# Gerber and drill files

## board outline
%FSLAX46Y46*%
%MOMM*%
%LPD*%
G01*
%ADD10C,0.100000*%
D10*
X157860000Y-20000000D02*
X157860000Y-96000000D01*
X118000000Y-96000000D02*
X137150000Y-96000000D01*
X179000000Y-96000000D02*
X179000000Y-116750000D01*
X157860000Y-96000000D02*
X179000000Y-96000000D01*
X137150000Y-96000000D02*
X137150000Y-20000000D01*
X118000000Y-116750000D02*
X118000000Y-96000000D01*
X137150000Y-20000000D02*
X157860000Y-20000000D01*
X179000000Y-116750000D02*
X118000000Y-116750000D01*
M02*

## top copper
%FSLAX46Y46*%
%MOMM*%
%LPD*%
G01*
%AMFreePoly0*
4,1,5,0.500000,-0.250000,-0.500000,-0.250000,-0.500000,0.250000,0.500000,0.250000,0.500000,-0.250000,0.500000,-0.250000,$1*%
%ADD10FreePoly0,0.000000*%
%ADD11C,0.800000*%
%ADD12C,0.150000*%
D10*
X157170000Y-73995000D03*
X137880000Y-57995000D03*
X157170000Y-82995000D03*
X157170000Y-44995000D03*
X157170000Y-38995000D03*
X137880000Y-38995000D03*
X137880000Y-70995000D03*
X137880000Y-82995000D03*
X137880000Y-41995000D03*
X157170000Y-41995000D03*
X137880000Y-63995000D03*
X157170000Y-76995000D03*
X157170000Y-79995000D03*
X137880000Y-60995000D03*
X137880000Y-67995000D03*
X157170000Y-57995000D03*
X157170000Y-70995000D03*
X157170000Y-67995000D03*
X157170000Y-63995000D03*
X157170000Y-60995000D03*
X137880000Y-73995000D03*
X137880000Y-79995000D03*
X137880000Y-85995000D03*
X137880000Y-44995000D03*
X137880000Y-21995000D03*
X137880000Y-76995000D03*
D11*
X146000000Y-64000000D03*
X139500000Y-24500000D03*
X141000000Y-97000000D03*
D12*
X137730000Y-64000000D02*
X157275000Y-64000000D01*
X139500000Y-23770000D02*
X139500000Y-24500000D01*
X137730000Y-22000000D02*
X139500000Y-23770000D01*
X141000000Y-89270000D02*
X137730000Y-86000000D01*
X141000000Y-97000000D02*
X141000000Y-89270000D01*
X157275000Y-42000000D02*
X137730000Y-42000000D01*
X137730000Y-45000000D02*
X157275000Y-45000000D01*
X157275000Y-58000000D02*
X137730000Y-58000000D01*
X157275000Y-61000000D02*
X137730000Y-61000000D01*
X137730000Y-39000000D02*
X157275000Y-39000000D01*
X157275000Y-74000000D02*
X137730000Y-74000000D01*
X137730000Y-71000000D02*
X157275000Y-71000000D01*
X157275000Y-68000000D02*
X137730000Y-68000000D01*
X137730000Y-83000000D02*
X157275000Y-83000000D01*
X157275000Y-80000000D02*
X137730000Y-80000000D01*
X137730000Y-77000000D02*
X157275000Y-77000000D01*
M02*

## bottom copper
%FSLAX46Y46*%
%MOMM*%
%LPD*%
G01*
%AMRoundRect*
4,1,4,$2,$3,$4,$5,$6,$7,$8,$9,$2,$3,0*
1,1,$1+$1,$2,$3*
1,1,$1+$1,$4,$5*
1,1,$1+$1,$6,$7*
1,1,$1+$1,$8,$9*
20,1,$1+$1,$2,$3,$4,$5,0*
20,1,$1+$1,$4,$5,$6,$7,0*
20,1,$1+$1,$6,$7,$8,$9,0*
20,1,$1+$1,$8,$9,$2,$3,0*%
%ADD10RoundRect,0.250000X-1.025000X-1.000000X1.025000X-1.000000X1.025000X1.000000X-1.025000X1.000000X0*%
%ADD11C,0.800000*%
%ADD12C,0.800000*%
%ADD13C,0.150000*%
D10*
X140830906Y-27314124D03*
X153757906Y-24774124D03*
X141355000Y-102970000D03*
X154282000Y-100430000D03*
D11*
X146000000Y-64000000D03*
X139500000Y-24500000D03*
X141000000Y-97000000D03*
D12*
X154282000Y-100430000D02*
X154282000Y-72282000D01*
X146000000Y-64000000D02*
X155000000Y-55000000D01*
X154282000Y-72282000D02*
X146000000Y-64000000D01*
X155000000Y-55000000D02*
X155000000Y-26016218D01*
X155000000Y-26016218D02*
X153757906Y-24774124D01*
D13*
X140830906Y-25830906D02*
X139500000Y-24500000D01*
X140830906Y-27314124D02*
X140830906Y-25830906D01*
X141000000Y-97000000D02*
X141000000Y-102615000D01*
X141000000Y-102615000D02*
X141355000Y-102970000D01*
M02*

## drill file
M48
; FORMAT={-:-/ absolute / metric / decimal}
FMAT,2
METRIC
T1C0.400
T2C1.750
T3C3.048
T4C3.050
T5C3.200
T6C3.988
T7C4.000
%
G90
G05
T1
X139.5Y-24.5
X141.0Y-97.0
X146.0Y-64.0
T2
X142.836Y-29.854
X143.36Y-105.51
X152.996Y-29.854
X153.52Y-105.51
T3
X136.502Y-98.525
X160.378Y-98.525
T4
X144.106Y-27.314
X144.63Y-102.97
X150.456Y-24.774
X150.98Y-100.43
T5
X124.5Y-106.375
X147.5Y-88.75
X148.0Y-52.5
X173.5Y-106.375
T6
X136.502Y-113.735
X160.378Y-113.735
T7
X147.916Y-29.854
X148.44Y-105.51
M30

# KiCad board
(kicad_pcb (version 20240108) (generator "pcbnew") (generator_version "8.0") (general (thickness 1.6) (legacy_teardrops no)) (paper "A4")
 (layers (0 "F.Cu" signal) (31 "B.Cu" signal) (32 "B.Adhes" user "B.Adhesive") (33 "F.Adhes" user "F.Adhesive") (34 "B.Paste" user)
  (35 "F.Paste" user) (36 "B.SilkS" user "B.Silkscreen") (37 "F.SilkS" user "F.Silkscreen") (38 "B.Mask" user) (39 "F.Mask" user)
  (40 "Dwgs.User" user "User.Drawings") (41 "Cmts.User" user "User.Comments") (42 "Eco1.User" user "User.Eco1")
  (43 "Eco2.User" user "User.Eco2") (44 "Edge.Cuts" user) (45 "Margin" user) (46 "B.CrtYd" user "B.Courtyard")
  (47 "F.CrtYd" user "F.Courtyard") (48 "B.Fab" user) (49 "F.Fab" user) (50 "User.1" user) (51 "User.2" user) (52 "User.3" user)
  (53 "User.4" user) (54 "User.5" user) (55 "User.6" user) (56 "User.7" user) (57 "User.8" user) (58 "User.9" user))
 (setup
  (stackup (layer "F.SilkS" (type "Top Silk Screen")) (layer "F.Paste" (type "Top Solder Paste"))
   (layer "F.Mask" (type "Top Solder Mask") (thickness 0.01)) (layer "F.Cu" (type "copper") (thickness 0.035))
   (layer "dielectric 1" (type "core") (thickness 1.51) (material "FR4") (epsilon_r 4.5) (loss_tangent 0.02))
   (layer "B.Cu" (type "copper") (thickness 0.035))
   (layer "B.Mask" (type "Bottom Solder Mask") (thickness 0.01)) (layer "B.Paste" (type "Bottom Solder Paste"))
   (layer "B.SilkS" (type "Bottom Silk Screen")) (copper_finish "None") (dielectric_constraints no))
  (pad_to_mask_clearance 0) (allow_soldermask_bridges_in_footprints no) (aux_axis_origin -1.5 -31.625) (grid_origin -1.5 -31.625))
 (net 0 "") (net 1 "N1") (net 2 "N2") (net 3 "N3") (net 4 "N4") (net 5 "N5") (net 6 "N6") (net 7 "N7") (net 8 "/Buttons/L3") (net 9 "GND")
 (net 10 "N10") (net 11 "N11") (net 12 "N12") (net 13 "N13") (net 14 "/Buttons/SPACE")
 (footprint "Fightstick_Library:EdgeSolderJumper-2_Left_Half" (layer "F.Cu") (at 157.82 73.995)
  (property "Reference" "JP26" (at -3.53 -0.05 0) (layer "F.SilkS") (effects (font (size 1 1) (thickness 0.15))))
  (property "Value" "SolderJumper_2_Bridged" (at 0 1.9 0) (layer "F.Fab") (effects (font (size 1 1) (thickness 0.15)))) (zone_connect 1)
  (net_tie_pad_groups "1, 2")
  (pad "1" smd custom (at -0.65 0) (size 1 0.5) (layers "F.Cu" "F.Mask") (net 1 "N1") (zone_connect 2) (thermal_bridge_angle 45)
   (options (clearance outline) (anchor rect)) (primitives)))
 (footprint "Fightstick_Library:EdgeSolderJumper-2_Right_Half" (layer "F.Cu") (at 137.23 57.995)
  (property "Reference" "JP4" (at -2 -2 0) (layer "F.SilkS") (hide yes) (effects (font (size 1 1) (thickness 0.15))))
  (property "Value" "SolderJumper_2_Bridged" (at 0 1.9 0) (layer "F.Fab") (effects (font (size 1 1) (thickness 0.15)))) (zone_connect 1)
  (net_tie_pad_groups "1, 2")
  (pad "2" smd custom (at 0.65 0) (size 1 0.5) (layers "F.Cu" "F.Mask") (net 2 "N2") (zone_connect 2) (thermal_bridge_angle 45)
   (options (clearance outline) (anchor rect)) (primitives)))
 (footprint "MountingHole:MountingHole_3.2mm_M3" (layer "F.Cu") (at 148 52.5 -90)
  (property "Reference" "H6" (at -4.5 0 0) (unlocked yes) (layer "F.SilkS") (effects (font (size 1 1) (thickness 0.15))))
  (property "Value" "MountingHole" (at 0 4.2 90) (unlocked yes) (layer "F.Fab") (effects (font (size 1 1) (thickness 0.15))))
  (pad "" np_thru_hole circle (at 0 0 270) (size 3.2 3.2) (drill 3.2) (layers "*.Cu" "*.Mask")))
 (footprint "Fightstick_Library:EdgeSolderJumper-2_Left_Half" (layer "F.Cu") (at 157.82 82.995)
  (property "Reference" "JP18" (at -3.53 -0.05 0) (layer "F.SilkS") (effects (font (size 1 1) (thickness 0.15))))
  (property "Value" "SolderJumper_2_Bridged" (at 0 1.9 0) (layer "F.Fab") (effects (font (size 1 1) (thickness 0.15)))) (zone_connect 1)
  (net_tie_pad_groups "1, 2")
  (pad "1" smd custom (at -0.65 0) (size 1 0.5) (layers "F.Cu" "F.Mask") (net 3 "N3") (zone_connect 2) (thermal_bridge_angle 45)
   (options (clearance outline) (anchor rect)) (primitives)))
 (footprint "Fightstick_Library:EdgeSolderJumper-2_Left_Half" (layer "F.Cu") (at 157.82 44.995)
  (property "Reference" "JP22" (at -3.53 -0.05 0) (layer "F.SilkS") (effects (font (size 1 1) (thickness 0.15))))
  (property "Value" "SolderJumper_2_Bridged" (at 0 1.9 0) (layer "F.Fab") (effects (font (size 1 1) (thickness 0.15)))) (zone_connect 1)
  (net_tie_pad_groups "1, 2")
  (pad "1" smd custom (at -0.65 0) (size 1 0.5) (layers "F.Cu" "F.Mask") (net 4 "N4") (zone_connect 2) (thermal_bridge_angle 45)
   (options (clearance outline) (anchor rect)) (primitives)))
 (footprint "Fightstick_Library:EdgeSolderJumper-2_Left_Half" (layer "F.Cu") (at 157.82 38.995)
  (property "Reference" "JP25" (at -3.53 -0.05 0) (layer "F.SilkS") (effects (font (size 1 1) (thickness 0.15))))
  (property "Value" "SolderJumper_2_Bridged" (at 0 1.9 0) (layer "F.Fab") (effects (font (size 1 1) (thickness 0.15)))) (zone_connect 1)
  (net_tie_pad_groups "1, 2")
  (pad "1" smd custom (at -0.65 0) (size 1 0.5) (layers "F.Cu" "F.Mask") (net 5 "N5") (zone_connect 2) (thermal_bridge_angle 45)
   (options (clearance outline) (anchor rect)) (primitives)))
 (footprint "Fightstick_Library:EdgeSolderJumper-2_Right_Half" (layer "F.Cu") (at 137.23 38.995)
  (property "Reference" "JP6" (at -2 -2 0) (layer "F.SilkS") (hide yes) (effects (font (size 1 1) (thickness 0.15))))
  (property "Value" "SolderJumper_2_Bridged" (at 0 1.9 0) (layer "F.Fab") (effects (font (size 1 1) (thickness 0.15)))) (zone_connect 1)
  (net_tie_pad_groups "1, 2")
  (pad "2" smd custom (at 0.65 0) (size 1 0.5) (layers "F.Cu" "F.Mask") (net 5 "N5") (zone_connect 2) (thermal_bridge_angle 45)
   (options (clearance outline) (anchor rect)) (primitives)))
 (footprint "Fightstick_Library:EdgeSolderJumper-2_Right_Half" (layer "F.Cu") (at 137.23 70.995)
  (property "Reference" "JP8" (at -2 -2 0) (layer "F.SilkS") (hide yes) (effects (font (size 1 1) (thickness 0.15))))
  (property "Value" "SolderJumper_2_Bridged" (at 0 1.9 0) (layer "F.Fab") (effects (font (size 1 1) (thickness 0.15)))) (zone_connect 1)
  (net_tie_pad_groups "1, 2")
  (pad "2" smd custom (at 0.65 0) (size 1 0.5) (layers "F.Cu" "F.Mask") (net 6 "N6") (zone_connect 2) (thermal_bridge_angle 45)
   (options (clearance outline) (anchor rect)) (primitives)))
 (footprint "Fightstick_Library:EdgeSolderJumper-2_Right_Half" (layer "F.Cu") (at 137.23 82.995)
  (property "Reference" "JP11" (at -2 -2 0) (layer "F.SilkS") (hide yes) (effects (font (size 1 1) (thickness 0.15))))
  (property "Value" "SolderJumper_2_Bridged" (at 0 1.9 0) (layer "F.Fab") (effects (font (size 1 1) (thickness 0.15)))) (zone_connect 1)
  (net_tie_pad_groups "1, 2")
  (pad "2" smd custom (at 0.65 0) (size 1 0.5) (layers "F.Cu" "F.Mask") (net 3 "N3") (zone_connect 2) (thermal_bridge_angle 45)
   (options (clearance outline) (anchor rect)) (primitives)))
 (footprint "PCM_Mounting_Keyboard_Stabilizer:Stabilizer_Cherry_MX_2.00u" (layer "F.Cu") (at 148.44 105.51)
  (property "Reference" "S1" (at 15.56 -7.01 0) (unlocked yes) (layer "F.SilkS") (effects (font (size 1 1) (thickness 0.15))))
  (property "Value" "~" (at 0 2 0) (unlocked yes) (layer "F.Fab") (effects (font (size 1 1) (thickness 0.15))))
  (pad "" np_thru_hole circle (at -11.938 -6.985) (size 3.048 3.048) (drill 3.048) (layers "*.Cu" "*.Mask"))
  (pad "" np_thru_hole circle (at -11.938 8.225) (size 3.9878 3.9878) (drill 3.9878) (layers "*.Cu" "*.Mask"))
  (pad "" np_thru_hole circle (at 11.938 -6.985) (size 3.048 3.048) (drill 3.048) (layers "*.Cu" "*.Mask"))
  (pad "" np_thru_hole circle (at 11.938 8.225) (size 3.9878 3.9878) (drill 3.9878) (layers "*.Cu" "*.Mask")))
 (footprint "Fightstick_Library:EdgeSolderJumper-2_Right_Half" (layer "F.Cu") (at 137.23 41.995)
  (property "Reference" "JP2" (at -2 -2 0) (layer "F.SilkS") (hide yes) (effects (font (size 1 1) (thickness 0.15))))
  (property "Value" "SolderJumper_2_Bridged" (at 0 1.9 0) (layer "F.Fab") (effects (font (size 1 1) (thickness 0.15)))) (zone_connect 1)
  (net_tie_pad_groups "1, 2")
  (pad "2" smd custom (at 0.65 0) (size 1 0.5) (layers "F.Cu" "F.Mask") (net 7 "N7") (zone_connect 2) (thermal_bridge_angle 45)
   (options (clearance outline) (anchor rect)) (primitives)))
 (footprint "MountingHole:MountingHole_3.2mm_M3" (layer "F.Cu") (at 147.5 88.75)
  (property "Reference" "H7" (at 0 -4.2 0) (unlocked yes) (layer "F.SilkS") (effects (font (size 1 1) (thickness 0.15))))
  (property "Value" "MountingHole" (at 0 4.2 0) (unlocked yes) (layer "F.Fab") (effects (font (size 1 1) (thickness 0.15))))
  (pad "" np_thru_hole circle (at 0 0) (size 3.2 3.2) (drill 3.2) (layers "*.Cu" "*.Mask")))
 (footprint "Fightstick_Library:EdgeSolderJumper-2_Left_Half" (layer "F.Cu") (at 157.82 41.995)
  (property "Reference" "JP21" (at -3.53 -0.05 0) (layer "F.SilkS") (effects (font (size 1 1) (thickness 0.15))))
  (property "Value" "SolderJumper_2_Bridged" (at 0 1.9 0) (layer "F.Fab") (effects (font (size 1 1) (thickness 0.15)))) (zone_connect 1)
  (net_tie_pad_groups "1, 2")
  (pad "1" smd custom (at -0.65 0) (size 1 0.5) (layers "F.Cu" "F.Mask") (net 7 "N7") (zone_connect 2) (thermal_bridge_angle 45)
   (options (clearance outline) (anchor rect)) (primitives)))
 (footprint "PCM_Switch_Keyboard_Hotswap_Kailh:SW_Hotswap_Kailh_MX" (layer "F.Cu") (at 147.915906 29.854124)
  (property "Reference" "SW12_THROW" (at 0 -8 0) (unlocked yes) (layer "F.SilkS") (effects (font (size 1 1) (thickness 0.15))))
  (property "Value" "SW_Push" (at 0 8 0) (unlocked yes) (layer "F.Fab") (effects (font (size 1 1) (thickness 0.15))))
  (pad "" np_thru_hole circle (at -5.08 0) (size 1.75 1.75) (drill 1.75) (layers "*.Cu" "*.Mask"))
  (pad "" np_thru_hole circle (at -3.81 -2.54) (size 3.05 3.05) (drill 3.05) (layers "*.Cu" "*.Mask"))
  (pad "" np_thru_hole circle (at 0 0) (size 4 4) (drill 4) (layers "*.Cu" "*.Mask"))
  (pad "" np_thru_hole circle (at 2.54 -5.08) (size 3.05 3.05) (drill 3.05) (layers "*.Cu" "*.Mask"))
  (pad "" np_thru_hole circle (at 5.08 0) (size 1.75 1.75) (drill 1.75) (layers "*.Cu" "*.Mask"))
  (pad "1" smd roundrect (at -7.085 -2.54) (size 2.55 2.5) (layers "B.Cu" "B.Paste" "B.Mask") (roundrect_rratio 0.1) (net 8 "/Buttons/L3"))
  (pad "2" smd roundrect (at 5.842 -5.08) (size 2.55 2.5) (layers "B.Cu" "B.Paste" "B.Mask") (roundrect_rratio 0.1) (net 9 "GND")))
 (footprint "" (layer "F.Cu") (at 173.5 106.375)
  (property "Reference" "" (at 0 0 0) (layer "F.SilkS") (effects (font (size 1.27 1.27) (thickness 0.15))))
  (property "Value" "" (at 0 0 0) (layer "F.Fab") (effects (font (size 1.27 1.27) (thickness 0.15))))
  (pad "" np_thru_hole circle (at 0 0 270) (size 3.2 3.2) (drill 3.2) (layers "F&B.Cu" "*.Mask")))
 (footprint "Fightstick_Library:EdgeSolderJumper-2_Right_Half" (layer "F.Cu") (at 137.23 63.995)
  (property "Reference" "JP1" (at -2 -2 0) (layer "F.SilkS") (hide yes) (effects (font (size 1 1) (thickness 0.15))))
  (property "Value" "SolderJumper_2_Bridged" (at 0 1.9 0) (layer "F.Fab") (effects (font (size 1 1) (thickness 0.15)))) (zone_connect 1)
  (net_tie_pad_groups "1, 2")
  (pad "2" smd custom (at 0.65 0) (size 1 0.5) (layers "F.Cu" "F.Mask") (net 9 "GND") (zone_connect 2) (thermal_bridge_angle 45)
   (options (clearance outline) (anchor rect)) (primitives)))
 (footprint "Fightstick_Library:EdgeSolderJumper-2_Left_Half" (layer "F.Cu") (at 157.82 76.995)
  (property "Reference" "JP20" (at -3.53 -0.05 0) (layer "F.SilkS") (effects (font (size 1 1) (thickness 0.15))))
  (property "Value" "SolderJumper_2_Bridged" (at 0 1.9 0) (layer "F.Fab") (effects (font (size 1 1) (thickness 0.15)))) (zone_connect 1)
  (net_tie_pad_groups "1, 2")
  (pad "1" smd custom (at -0.65 0) (size 1 0.5) (layers "F.Cu" "F.Mask") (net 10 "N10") (zone_connect 2) (thermal_bridge_angle 45)
   (options (clearance outline) (anchor rect)) (primitives)))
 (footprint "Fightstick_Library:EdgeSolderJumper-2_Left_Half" (layer "F.Cu") (at 157.82 79.995)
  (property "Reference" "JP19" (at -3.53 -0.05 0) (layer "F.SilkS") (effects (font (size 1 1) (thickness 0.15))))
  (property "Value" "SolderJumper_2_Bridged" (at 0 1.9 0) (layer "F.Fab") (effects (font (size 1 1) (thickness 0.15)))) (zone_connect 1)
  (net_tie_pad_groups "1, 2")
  (pad "1" smd custom (at -0.65 0) (size 1 0.5) (layers "F.Cu" "F.Mask") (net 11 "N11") (zone_connect 2) (thermal_bridge_angle 45)
   (options (clearance outline) (anchor rect)) (primitives)))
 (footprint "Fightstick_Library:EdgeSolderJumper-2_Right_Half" (layer "F.Cu") (at 137.23 60.995)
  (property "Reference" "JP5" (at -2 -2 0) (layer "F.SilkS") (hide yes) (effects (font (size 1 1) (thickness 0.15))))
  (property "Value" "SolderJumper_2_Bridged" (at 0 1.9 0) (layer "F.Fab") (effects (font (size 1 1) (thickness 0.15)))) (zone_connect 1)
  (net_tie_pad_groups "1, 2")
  (pad "2" smd custom (at 0.65 0) (size 1 0.5) (layers "F.Cu" "F.Mask") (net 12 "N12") (zone_connect 2) (thermal_bridge_angle 45)
   (options (clearance outline) (anchor rect)) (primitives)))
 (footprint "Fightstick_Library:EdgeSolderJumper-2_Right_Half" (layer "F.Cu") (at 137.23 67.995)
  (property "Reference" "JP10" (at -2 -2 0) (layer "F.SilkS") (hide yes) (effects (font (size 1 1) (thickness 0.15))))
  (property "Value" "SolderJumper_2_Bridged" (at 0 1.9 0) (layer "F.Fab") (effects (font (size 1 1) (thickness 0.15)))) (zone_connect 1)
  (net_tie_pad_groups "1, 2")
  (pad "2" smd custom (at 0.65 0) (size 1 0.5) (layers "F.Cu" "F.Mask") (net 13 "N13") (zone_connect 2) (thermal_bridge_angle 45)
   (options (clearance outline) (anchor rect)) (primitives)))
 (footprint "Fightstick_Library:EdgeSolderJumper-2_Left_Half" (layer "F.Cu") (at 157.82 57.995)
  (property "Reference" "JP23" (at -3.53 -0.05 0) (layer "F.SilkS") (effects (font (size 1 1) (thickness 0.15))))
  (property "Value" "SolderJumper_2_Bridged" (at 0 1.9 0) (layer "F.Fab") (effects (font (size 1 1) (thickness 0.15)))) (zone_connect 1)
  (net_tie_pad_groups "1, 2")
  (pad "1" smd custom (at -0.65 0) (size 1 0.5) (layers "F.Cu" "F.Mask") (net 2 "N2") (zone_connect 2) (thermal_bridge_angle 45)
   (options (clearance outline) (anchor rect)) (primitives)))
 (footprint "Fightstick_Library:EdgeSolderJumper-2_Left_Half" (layer "F.Cu") (at 157.82 70.995)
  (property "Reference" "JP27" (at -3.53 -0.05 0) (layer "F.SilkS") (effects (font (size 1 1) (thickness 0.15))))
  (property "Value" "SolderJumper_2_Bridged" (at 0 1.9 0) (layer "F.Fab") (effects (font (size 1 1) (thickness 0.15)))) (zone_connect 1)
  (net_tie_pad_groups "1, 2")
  (pad "1" smd custom (at -0.65 0) (size 1 0.5) (layers "F.Cu" "F.Mask") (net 6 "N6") (zone_connect 2) (thermal_bridge_angle 45)
   (options (clearance outline) (anchor rect)) (primitives)))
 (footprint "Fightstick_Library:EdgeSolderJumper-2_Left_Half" (layer "F.Cu") (at 157.82 67.995)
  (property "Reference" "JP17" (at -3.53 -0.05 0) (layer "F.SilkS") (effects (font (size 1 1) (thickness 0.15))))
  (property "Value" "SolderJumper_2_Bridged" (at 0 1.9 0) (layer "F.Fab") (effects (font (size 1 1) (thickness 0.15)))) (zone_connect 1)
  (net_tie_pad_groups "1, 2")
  (pad "1" smd custom (at -0.65 0) (size 1 0.5) (layers "F.Cu" "F.Mask") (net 13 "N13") (zone_connect 2) (thermal_bridge_angle 45)
   (options (clearance outline) (anchor rect)) (primitives)))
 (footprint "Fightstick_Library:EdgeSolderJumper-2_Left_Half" (layer "F.Cu") (at 157.82 63.995)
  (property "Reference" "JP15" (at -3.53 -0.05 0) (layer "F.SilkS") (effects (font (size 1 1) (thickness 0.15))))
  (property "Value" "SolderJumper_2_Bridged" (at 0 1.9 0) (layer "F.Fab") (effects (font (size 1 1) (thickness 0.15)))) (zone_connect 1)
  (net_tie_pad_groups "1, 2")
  (pad "1" smd custom (at -0.65 0) (size 1 0.5) (layers "F.Cu" "F.Mask") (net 9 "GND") (zone_connect 2) (thermal_bridge_angle 45)
   (options (clearance outline) (anchor rect)) (primitives)))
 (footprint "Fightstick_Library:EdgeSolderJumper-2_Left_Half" (layer "F.Cu") (at 157.82 60.995)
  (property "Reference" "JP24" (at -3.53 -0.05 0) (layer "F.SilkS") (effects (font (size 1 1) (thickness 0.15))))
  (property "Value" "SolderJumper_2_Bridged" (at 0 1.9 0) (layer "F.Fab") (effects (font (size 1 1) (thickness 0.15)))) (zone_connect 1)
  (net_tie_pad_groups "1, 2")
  (pad "1" smd custom (at -0.65 0) (size 1 0.5) (layers "F.Cu" "F.Mask") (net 12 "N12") (zone_connect 2) (thermal_bridge_angle 45)
   (options (clearance outline) (anchor rect)) (primitives)))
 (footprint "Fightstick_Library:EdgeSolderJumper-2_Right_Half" (layer "F.Cu") (at 137.23 73.995)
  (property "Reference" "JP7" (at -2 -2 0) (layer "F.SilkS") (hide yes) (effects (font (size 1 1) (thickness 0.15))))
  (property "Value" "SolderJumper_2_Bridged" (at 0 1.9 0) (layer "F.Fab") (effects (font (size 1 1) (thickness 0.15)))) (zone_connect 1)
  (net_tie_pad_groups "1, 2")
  (pad "2" smd custom (at 0.65 0) (size 1 0.5) (layers "F.Cu" "F.Mask") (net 1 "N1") (zone_connect 2) (thermal_bridge_angle 45)
   (options (clearance outline) (anchor rect)) (primitives)))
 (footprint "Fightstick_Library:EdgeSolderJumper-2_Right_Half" (layer "F.Cu") (at 137.23 79.995)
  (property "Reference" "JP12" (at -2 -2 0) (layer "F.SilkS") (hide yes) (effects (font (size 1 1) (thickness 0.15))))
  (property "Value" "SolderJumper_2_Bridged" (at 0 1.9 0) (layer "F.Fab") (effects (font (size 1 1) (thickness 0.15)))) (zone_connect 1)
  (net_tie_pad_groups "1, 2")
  (pad "2" smd custom (at 0.65 0) (size 1 0.5) (layers "F.Cu" "F.Mask") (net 11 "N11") (zone_connect 2) (thermal_bridge_angle 45)
   (options (clearance outline) (anchor rect)) (primitives)))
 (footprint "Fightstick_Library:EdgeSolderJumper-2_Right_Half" (layer "F.Cu") (at 137.23 85.995)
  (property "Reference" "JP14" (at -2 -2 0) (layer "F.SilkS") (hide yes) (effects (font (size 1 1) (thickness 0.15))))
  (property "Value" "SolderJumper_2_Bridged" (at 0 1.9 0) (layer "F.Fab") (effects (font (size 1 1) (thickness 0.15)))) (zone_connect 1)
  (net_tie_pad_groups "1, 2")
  (pad "2" smd custom (at 0.65 0) (size 1 0.5) (layers "F.Cu" "F.Mask") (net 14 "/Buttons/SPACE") (zone_connect 2) (thermal_bridge_angle 45)
   (options (clearance outline) (anchor rect)) (primitives)))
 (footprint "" (layer "F.Cu") (at 124.5 106.375)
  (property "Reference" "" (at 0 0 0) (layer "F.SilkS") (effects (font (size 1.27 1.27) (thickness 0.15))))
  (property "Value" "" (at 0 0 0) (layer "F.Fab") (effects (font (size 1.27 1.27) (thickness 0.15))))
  (pad "" np_thru_hole circle (at 0 0 270) (size 3.2 3.2) (drill 3.2) (layers "F&B.Cu" "*.Mask")))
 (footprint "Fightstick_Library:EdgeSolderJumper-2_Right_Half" (layer "F.Cu") (at 137.23 44.995)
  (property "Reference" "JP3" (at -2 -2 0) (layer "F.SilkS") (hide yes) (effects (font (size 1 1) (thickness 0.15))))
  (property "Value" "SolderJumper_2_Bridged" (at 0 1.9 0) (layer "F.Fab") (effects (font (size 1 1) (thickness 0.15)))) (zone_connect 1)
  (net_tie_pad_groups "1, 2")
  (pad "2" smd custom (at 0.65 0) (size 1 0.5) (layers "F.Cu" "F.Mask") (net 4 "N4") (zone_connect 2) (thermal_bridge_angle 45)
   (options (clearance outline) (anchor rect)) (primitives)))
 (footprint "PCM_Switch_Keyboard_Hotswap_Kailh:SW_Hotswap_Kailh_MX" (layer "F.Cu") (at 148.44 105.51)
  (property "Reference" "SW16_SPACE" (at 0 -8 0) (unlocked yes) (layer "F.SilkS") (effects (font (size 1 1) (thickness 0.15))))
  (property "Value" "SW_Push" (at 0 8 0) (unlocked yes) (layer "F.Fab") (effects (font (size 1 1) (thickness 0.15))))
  (pad "" np_thru_hole circle (at -5.08 0) (size 1.75 1.75) (drill 1.75) (layers "*.Cu" "*.Mask"))
  (pad "" np_thru_hole circle (at -3.81 -2.54) (size 3.05 3.05) (drill 3.05) (layers "*.Cu" "*.Mask"))
  (pad "" np_thru_hole circle (at 0 0) (size 4 4) (drill 4) (layers "*.Cu" "*.Mask"))
  (pad "" np_thru_hole circle (at 2.54 -5.08) (size 3.05 3.05) (drill 3.05) (layers "*.Cu" "*.Mask"))
  (pad "" np_thru_hole circle (at 5.08 0) (size 1.75 1.75) (drill 1.75) (layers "*.Cu" "*.Mask"))
  (pad "1" smd roundrect (at -7.085 -2.54) (size 2.55 2.5) (layers "B.Cu" "B.Paste" "B.Mask") (roundrect_rratio 0.1)
   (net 14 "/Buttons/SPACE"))
  (pad "2" smd roundrect (at 5.842 -5.08) (size 2.55 2.5) (layers "B.Cu" "B.Paste" "B.Mask") (roundrect_rratio 0.1) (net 9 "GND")))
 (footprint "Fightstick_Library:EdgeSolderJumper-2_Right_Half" (layer "F.Cu") (at 137.23 21.995)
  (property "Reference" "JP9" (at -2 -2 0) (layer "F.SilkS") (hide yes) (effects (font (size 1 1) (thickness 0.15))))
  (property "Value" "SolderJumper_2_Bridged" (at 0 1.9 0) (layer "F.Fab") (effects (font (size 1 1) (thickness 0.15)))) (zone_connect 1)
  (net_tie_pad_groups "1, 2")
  (pad "2" smd custom (at 0.65 0) (size 1 0.5) (layers "F.Cu" "F.Mask") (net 8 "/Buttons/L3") (zone_connect 2) (thermal_bridge_angle 45)
   (options (clearance outline) (anchor rect)) (primitives)))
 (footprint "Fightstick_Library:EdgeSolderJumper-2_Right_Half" (layer "F.Cu") (at 137.23 76.995)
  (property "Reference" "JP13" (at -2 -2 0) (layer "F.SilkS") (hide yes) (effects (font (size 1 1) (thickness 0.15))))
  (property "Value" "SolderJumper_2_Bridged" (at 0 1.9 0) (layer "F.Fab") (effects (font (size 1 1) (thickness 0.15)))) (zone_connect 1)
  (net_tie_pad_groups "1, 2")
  (pad "2" smd custom (at 0.65 0) (size 1 0.5) (layers "F.Cu" "F.Mask") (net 10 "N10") (zone_connect 2) (thermal_bridge_angle 45)
   (options (clearance outline) (anchor rect)) (primitives)))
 (gr_line (start 157.86 20) (end 157.86 96) (stroke (width 0.1) (type default)) (layer "Edge.Cuts"))
 (gr_line (start 118 96) (end 137.15 96) (stroke (width 0.1) (type default)) (layer "Edge.Cuts"))
 (gr_line (start 179 96) (end 179 116.75) (stroke (width 0.1) (type default)) (layer "Edge.Cuts"))
 (gr_line (start 157.86 96) (end 179 96) (stroke (width 0.1) (type default)) (layer "Edge.Cuts"))
 (gr_line (start 137.15 96) (end 137.15 20) (stroke (width 0.1) (type default)) (layer "Edge.Cuts"))
 (gr_line (start 118 116.75) (end 118 96) (stroke (width 0.1) (type default)) (layer "Edge.Cuts"))
 (gr_line (start 137.15 20) (end 157.86 20) (stroke (width 0.1) (type default)) (layer "Edge.Cuts"))
 (gr_line (start 179 116.75) (end 118 116.75) (stroke (width 0.1) (type default)) (layer "Edge.Cuts"))
 (segment (start 137.73 64) (end 157.275 64) (width 0.15) (layer "F.Cu") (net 9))
 (via (at 146 64) (size 0.8) (drill 0.4) (layers "F.Cu" "B.Cu") (free yes) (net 9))
 (segment (start 154.282 100.43) (end 154.282 72.282) (width 0.8) (layer "B.Cu") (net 9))
 (segment (start 146 64) (end 155 55) (width 0.8) (layer "B.Cu") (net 9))
 (segment (start 154.282 72.282) (end 146 64) (width 0.8) (layer "B.Cu") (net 9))
 (segment (start 155 55) (end 155 26.016218) (width 0.8) (layer "B.Cu") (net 9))
 (segment (start 155 26.016218) (end 153.757906 24.774124) (width 0.8) (layer "B.Cu") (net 9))
 (segment (start 139.5 23.77) (end 139.5 24.5) (width 0.15) (layer "F.Cu") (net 8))
 (segment (start 137.73 22) (end 139.5 23.77) (width 0.15) (layer "F.Cu") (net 8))
 (via (at 139.5 24.5) (size 0.8) (drill 0.4) (layers "F.Cu" "B.Cu") (free yes) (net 8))
 (segment (start 140.830906 25.830906) (end 139.5 24.5) (width 0.15) (layer "B.Cu") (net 8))
 (segment (start 140.830906 27.314124) (end 140.830906 25.830906) (width 0.15) (layer "B.Cu") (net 8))
 (segment (start 141 89.27) (end 137.73 86) (width 0.15) (layer "F.Cu") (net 14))
 (segment (start 141 97) (end 141 89.27) (width 0.15) (layer "F.Cu") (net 14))
 (via (at 141 97) (size 0.8) (drill 0.4) (layers "F.Cu" "B.Cu") (free yes) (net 14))
 (segment (start 141 97) (end 141 102.615) (width 0.15) (layer "B.Cu") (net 14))
 (segment (start 141 102.615) (end 141.355 102.97) (width 0.15) (layer "B.Cu") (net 14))
 (segment (start 157.275 42) (end 137.73 42) (width 0.15) (layer "F.Cu") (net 7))
 (segment (start 137.73 45) (end 157.275 45) (width 0.15) (layer "F.Cu") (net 4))
 (segment (start 157.275 58) (end 137.73 58) (width 0.15) (layer "F.Cu") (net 2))
 (segment (start 157.275 61) (end 137.73 61) (width 0.15) (layer "F.Cu") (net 12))
 (segment (start 137.73 39) (end 157.275 39) (width 0.15) (layer "F.Cu") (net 5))
 (segment (start 157.275 74) (end 137.73 74) (width 0.15) (layer "F.Cu") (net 1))
 (segment (start 137.73 71) (end 157.275 71) (width 0.15) (layer "F.Cu") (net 6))
 (segment (start 157.275 68) (end 137.73 68) (width 0.15) (layer "F.Cu") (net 13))
 (segment (start 137.73 83) (end 157.275 83) (width 0.15) (layer "F.Cu") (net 3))
 (segment (start 157.275 80) (end 137.73 80) (width 0.15) (layer "F.Cu") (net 11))
 (segment (start 137.73 77) (end 157.275 77) (width 0.15) (layer "F.Cu") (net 10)))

